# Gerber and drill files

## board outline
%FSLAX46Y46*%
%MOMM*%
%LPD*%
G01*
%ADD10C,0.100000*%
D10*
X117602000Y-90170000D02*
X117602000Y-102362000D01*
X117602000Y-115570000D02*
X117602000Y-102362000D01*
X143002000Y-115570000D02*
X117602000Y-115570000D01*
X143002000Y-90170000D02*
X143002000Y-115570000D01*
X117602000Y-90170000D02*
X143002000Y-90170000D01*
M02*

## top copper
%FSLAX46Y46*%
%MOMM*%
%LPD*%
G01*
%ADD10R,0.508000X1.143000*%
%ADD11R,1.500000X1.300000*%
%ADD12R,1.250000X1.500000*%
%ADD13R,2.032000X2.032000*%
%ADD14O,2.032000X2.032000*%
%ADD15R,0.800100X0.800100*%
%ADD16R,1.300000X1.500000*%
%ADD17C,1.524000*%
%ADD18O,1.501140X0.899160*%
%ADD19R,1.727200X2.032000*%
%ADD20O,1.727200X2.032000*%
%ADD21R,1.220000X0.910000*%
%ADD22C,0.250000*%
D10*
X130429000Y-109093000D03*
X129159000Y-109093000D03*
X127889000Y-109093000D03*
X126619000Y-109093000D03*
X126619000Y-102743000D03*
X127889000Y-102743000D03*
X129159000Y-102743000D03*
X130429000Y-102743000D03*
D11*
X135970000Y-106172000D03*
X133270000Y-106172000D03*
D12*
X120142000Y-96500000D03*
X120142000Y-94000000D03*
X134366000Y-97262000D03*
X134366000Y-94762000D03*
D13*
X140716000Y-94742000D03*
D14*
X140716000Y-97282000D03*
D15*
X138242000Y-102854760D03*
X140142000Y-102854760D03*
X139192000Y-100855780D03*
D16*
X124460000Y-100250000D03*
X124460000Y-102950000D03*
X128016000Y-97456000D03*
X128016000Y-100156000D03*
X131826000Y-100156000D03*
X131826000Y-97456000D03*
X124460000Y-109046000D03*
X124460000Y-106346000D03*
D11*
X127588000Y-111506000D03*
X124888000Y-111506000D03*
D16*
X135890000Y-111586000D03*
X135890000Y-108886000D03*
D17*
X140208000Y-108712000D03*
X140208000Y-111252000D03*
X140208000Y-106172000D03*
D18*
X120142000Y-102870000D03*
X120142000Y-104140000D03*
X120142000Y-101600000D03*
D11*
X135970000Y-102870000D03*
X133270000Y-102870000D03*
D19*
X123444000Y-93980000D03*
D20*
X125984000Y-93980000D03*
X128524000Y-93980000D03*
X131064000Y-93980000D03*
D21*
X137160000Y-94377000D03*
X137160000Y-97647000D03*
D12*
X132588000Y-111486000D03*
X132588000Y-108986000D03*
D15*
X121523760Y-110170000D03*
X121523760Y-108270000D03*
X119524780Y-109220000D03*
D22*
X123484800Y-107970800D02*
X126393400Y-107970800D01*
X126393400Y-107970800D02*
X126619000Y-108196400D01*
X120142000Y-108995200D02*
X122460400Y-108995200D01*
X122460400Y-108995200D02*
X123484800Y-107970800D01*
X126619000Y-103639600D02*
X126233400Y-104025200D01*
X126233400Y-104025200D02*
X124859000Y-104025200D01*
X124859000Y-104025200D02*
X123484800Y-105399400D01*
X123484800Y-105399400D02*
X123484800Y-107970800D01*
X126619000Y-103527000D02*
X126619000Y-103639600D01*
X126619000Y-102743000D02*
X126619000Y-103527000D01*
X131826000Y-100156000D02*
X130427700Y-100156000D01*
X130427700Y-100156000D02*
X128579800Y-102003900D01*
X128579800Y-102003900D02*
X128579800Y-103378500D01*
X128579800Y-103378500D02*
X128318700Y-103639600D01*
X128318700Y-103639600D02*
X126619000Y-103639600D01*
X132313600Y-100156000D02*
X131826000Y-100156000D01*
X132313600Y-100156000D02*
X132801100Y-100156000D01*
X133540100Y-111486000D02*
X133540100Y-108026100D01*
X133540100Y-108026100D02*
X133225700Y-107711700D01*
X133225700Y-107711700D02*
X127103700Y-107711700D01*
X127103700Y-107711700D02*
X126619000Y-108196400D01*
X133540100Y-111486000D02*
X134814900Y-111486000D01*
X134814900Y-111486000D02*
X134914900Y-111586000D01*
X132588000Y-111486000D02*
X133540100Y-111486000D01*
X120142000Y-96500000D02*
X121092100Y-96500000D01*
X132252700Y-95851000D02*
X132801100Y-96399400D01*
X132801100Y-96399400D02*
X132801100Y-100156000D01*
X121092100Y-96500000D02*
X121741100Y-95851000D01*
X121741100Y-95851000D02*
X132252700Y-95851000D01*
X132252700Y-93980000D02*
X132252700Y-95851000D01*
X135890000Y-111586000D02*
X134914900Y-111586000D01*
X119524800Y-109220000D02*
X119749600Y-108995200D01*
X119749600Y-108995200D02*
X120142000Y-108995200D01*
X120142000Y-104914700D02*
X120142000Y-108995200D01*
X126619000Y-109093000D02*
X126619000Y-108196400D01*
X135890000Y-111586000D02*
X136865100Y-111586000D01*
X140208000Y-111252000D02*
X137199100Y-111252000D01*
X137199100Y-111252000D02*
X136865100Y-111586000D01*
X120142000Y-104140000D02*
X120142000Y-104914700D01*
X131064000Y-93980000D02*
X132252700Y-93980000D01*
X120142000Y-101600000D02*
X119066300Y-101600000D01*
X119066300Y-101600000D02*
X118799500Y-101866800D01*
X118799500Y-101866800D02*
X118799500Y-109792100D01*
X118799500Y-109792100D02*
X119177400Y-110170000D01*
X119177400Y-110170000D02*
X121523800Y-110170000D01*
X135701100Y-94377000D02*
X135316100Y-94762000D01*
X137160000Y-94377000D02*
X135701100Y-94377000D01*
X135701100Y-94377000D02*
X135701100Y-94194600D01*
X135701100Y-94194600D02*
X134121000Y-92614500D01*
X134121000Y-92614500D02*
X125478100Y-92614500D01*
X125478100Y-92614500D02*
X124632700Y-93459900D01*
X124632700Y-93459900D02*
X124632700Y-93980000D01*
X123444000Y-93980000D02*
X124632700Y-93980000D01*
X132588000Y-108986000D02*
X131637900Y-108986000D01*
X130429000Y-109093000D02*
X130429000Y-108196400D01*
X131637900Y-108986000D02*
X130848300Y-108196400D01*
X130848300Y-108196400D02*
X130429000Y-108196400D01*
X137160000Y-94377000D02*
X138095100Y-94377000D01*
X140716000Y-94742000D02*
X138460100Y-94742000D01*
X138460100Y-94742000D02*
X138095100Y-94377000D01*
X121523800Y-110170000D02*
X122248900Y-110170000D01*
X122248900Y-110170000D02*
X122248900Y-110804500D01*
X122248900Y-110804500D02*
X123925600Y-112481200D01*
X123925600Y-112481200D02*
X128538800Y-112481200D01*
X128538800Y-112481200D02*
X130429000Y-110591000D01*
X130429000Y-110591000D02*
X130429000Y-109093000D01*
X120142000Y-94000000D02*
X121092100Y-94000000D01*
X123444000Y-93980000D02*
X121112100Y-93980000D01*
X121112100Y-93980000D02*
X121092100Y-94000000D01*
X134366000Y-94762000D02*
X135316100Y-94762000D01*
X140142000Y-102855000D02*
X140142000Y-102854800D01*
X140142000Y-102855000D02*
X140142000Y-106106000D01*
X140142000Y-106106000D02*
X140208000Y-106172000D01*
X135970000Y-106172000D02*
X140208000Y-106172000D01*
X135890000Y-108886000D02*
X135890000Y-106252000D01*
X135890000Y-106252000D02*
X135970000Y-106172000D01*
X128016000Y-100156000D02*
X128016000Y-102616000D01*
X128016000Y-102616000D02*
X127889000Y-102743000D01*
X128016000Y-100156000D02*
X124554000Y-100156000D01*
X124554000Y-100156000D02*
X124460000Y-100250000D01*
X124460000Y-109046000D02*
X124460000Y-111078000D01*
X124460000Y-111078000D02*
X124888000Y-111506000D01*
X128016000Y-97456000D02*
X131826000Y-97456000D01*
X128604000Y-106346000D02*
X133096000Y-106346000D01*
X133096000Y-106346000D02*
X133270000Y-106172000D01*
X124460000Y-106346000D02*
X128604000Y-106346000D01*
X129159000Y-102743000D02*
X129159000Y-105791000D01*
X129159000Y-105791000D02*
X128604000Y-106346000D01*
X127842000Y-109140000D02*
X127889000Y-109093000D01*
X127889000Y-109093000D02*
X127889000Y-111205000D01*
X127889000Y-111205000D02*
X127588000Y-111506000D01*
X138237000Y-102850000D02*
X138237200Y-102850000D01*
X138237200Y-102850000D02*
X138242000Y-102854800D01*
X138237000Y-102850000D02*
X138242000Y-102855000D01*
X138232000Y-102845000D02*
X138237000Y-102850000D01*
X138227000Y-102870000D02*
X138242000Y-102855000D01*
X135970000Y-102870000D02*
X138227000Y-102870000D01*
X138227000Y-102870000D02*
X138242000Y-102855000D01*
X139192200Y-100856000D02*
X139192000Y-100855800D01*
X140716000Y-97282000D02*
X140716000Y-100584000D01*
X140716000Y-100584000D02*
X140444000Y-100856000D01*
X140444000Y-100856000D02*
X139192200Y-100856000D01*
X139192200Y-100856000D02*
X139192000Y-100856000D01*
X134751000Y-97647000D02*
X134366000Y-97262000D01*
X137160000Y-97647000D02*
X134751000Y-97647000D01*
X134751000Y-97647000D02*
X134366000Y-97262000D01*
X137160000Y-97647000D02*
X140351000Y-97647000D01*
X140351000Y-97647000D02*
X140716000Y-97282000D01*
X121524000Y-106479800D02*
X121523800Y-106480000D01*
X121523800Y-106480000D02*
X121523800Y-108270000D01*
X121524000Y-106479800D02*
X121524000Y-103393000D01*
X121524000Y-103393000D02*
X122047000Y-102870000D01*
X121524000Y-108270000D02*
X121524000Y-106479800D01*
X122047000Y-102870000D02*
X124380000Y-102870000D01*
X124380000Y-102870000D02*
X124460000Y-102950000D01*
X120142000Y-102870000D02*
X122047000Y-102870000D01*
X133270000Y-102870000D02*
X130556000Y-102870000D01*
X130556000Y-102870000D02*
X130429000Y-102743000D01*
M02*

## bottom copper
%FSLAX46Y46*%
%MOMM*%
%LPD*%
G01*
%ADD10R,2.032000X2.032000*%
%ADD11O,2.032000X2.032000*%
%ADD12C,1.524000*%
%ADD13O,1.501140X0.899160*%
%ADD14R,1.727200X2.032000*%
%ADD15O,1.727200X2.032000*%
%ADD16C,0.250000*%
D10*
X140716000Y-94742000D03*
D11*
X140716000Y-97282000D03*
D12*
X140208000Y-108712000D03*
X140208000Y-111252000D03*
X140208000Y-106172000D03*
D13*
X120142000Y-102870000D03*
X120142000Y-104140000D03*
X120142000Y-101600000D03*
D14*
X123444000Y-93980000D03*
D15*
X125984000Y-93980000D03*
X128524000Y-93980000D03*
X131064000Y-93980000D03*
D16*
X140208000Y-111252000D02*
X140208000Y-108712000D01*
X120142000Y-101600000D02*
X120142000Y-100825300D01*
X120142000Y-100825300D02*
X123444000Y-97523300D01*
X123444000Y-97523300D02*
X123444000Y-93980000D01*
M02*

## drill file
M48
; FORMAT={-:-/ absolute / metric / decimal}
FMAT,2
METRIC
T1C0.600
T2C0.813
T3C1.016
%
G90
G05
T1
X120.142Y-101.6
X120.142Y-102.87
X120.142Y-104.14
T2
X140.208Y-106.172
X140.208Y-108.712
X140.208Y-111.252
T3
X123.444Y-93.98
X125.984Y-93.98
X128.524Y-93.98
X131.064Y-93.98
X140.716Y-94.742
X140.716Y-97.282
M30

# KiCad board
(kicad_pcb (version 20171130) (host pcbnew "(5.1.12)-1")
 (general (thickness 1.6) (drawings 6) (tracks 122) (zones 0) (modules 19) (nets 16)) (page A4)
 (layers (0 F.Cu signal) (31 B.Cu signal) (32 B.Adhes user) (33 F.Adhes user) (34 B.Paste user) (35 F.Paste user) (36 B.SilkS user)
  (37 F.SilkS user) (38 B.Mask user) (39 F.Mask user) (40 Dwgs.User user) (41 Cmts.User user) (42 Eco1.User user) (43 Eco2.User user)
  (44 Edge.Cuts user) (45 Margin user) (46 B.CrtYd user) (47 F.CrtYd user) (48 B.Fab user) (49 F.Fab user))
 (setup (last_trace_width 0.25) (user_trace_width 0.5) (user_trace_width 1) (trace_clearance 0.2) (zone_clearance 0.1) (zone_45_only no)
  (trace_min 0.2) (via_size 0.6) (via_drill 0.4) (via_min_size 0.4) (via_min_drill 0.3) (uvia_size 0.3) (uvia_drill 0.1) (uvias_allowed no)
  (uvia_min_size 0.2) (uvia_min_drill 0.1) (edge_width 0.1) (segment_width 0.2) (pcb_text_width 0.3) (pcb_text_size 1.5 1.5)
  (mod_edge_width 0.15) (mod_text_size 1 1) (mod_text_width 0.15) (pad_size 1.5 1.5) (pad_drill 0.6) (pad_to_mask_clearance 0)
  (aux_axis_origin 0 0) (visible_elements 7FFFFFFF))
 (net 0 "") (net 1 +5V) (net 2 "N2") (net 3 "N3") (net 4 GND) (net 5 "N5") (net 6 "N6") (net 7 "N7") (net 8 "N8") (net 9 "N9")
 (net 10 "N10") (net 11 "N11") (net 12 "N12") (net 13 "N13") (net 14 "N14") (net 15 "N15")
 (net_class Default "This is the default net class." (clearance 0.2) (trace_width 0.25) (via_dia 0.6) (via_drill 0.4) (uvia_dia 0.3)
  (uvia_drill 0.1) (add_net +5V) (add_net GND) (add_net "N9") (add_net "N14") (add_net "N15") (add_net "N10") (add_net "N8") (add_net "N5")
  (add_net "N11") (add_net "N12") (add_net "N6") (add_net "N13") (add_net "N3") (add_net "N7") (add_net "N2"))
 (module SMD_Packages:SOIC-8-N (layer F.Cu) (at 128.524 105.918 180)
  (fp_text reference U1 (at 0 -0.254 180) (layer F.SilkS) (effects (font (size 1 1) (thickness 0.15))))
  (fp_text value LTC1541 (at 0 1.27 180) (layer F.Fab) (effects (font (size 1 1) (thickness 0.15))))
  (pad 8 smd rect (at -1.905 -3.175 180) (size 0.508 1.143) (layers F.Cu F.Paste F.Mask) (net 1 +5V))
  (pad 7 smd rect (at -0.635 -3.175 180) (size 0.508 1.143) (layers F.Cu F.Paste F.Mask) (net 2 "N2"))
  (pad 6 smd rect (at 0.635 -3.175 180) (size 0.508 1.143) (layers F.Cu F.Paste F.Mask) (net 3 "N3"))
  (pad 5 smd rect (at 1.905 -3.175 180) (size 0.508 1.143) (layers F.Cu F.Paste F.Mask) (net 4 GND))
  (pad 4 smd rect (at 1.905 3.175 180) (size 0.508 1.143) (layers F.Cu F.Paste F.Mask) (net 4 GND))
  (pad 3 smd rect (at 0.635 3.175 180) (size 0.508 1.143) (layers F.Cu F.Paste F.Mask) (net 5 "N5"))
  (pad 2 smd rect (at -0.635 3.175 180) (size 0.508 1.143) (layers F.Cu F.Paste F.Mask) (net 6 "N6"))
  (pad 1 smd rect (at -1.905 3.175 180) (size 0.508 1.143) (layers F.Cu F.Paste F.Mask) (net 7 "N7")))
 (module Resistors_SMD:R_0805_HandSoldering (layer F.Cu) (at 134.62 106.172 180)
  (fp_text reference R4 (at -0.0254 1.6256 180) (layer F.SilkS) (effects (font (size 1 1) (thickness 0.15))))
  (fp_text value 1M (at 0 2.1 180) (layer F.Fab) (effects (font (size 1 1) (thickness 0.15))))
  (pad 1 smd rect (at -1.35 0 180) (size 1.5 1.3) (layers F.Cu F.Paste F.Mask) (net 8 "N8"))
  (pad 2 smd rect (at 1.35 0 180) (size 1.5 1.3) (layers F.Cu F.Paste F.Mask) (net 6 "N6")))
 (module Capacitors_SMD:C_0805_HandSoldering (layer F.Cu) (at 120.142 95.25 90)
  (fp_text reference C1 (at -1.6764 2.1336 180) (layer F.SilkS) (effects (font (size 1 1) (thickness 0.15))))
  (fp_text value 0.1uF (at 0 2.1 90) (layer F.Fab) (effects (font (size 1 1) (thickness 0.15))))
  (pad 1 smd rect (at -1.25 0 90) (size 1.5 1.25) (layers F.Cu F.Paste F.Mask) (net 4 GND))
  (pad 2 smd rect (at 1.25 0 90) (size 1.5 1.25) (layers F.Cu F.Paste F.Mask) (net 1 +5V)))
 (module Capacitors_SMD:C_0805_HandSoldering (layer F.Cu) (at 134.366 96.012 90)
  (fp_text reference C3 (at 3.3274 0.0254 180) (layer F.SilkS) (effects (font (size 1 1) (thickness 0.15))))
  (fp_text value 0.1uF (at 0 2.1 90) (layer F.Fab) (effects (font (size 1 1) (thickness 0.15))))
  (pad 1 smd rect (at -1.25 0 90) (size 1.5 1.25) (layers F.Cu F.Paste F.Mask) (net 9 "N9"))
  (pad 2 smd rect (at 1.25 0 90) (size 1.5 1.25) (layers F.Cu F.Paste F.Mask) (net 1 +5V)))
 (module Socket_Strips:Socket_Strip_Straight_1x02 (layer F.Cu) (at 140.716 94.742 270)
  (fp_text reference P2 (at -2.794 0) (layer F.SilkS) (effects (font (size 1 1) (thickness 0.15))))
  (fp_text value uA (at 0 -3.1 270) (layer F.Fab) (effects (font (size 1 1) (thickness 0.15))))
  (pad 1 thru_hole rect (at 0 0 270) (size 2.032 2.032) (drill 1.016) (layers *.Cu *.Mask F.SilkS) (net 1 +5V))
  (pad 2 thru_hole oval (at 2.54 0 270) (size 2.032 2.032) (drill 1.016) (layers *.Cu *.Mask F.SilkS) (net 9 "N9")))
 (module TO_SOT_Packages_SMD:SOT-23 (layer F.Cu) (at 139.192 101.854)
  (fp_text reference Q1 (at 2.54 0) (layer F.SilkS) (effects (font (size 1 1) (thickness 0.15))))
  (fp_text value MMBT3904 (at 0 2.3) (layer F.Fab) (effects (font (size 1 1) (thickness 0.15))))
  (pad 1 smd rect (at -0.95 1.00076) (size 0.8001 0.8001) (layers F.Cu F.Paste F.Mask) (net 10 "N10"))
  (pad 2 smd rect (at 0.95 1.00076) (size 0.8001 0.8001) (layers F.Cu F.Paste F.Mask) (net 8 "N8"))
  (pad 3 smd rect (at 0 -0.99822) (size 0.8001 0.8001) (layers F.Cu F.Paste F.Mask) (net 9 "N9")))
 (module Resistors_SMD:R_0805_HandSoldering (layer F.Cu) (at 124.46 101.6 270)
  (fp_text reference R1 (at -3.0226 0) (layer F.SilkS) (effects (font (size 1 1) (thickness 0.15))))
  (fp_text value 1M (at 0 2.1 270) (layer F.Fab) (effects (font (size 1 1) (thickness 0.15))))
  (pad 1 smd rect (at -1.35 0 270) (size 1.5 1.3) (layers F.Cu F.Paste F.Mask) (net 5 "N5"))
  (pad 2 smd rect (at 1.35 0 270) (size 1.5 1.3) (layers F.Cu F.Paste F.Mask) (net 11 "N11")))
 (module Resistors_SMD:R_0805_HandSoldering (layer F.Cu) (at 128.016 98.806 270)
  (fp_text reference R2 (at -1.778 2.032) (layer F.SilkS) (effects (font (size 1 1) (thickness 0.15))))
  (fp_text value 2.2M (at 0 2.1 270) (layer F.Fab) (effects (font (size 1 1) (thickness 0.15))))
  (pad 1 smd rect (at -1.35 0 270) (size 1.5 1.3) (layers F.Cu F.Paste F.Mask) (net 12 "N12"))
  (pad 2 smd rect (at 1.35 0 270) (size 1.5 1.3) (layers F.Cu F.Paste F.Mask) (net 5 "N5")))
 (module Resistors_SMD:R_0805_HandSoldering (layer F.Cu) (at 131.826 98.806 90)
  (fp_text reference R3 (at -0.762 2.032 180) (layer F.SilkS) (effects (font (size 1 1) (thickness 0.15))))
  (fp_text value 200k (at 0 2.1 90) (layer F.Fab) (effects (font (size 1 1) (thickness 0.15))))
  (pad 1 smd rect (at -1.35 0 90) (size 1.5 1.3) (layers F.Cu F.Paste F.Mask) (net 4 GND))
  (pad 2 smd rect (at 1.35 0 90) (size 1.5 1.3) (layers F.Cu F.Paste F.Mask) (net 12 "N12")))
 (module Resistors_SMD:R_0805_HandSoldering (layer F.Cu) (at 124.46 107.696 90)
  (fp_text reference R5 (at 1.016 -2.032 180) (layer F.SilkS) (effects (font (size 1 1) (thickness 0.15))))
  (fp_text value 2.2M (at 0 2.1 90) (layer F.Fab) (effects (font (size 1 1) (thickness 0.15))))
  (pad 1 smd rect (at -1.35 0 90) (size 1.5 1.3) (layers F.Cu F.Paste F.Mask) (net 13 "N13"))
  (pad 2 smd rect (at 1.35 0 90) (size 1.5 1.3) (layers F.Cu F.Paste F.Mask) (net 6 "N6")))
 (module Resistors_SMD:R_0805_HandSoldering (layer F.Cu) (at 126.238 111.506 180)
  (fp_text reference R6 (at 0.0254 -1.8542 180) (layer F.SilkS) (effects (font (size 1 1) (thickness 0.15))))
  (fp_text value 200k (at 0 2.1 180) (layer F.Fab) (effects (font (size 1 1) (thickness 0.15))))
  (pad 1 smd rect (at -1.35 0 180) (size 1.5 1.3) (layers F.Cu F.Paste F.Mask) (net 3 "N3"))
  (pad 2 smd rect (at 1.35 0 180) (size 1.5 1.3) (layers F.Cu F.Paste F.Mask) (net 13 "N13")))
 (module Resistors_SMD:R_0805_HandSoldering (layer F.Cu) (at 135.89 110.236 90)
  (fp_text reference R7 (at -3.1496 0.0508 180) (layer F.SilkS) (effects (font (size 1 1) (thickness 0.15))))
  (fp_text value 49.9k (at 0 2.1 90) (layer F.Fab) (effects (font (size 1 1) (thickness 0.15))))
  (pad 1 smd rect (at -1.35 0 90) (size 1.5 1.3) (layers F.Cu F.Paste F.Mask) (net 4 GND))
  (pad 2 smd rect (at 1.35 0 90) (size 1.5 1.3) (layers F.Cu F.Paste F.Mask) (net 8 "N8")))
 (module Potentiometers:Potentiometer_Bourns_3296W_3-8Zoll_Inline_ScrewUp (layer F.Cu) (at 140.208 106.172 180)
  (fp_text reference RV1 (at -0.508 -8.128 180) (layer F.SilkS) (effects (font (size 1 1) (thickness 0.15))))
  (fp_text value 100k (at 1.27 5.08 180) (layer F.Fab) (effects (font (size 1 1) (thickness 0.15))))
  (pad 2 thru_hole circle (at 0 -2.54 180) (size 1.524 1.524) (drill 0.8128) (layers *.Cu *.Mask F.SilkS) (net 4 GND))
  (pad 3 thru_hole circle (at 0 -5.08 180) (size 1.524 1.524) (drill 0.8128) (layers *.Cu *.Mask F.SilkS) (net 4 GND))
  (pad 1 thru_hole circle (at 0 0 180) (size 1.524 1.524) (drill 0.8128) (layers *.Cu *.Mask F.SilkS) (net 8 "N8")))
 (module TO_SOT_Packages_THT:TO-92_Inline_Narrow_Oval (layer F.Cu) (at 120.142 101.6 270)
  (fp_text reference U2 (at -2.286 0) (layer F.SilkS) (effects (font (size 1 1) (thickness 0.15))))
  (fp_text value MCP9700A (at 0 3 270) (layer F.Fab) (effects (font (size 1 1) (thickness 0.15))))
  (pad 2 thru_hole oval (at 1.27 0 90) (size 0.89916 1.50114) (drill 0.6) (layers *.Cu *.Mask F.SilkS) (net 11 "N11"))
  (pad 3 thru_hole oval (at 2.54 0 90) (size 0.89916 1.50114) (drill 0.6) (layers *.Cu *.Mask F.SilkS) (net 4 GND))
  (pad 1 thru_hole oval (at 0 0 90) (size 0.89916 1.50114) (drill 0.6) (layers *.Cu *.Mask F.SilkS) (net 1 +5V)))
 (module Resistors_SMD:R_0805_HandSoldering (layer F.Cu) (at 134.62 102.87 180)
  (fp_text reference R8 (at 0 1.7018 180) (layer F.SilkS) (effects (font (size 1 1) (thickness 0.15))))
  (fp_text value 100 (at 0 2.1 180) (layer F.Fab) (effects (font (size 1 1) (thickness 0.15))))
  (pad 1 smd rect (at -1.35 0 180) (size 1.5 1.3) (layers F.Cu F.Paste F.Mask) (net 10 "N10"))
  (pad 2 smd rect (at 1.35 0 180) (size 1.5 1.3) (layers F.Cu F.Paste F.Mask) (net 7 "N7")))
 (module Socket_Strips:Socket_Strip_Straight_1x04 (layer F.Cu) (at 123.444 93.98)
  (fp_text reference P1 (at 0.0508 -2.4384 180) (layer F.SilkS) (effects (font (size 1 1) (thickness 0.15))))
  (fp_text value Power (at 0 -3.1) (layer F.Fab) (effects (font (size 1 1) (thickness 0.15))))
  (pad 1 thru_hole rect (at 0 0) (size 1.7272 2.032) (drill 1.016) (layers *.Cu *.Mask F.SilkS) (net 1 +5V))
  (pad 2 thru_hole oval (at 2.54 0) (size 1.7272 2.032) (drill 1.016) (layers *.Cu *.Mask F.SilkS) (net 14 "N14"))
  (pad 3 thru_hole oval (at 5.08 0) (size 1.7272 2.032) (drill 1.016) (layers *.Cu *.Mask F.SilkS) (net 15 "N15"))
  (pad 4 thru_hole oval (at 7.62 0) (size 1.7272 2.032) (drill 1.016) (layers *.Cu *.Mask F.SilkS) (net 4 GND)))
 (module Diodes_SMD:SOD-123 (layer F.Cu) (at 137.16 96.012 270)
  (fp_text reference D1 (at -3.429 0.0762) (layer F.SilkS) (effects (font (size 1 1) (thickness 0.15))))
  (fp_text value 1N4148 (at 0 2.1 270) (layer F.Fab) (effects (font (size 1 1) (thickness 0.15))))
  (pad 1 smd rect (at -1.635 0 270) (size 0.91 1.22) (layers F.Cu F.Paste F.Mask) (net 1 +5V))
  (pad 2 smd rect (at 1.635 0 270) (size 0.91 1.22) (layers F.Cu F.Paste F.Mask) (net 9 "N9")))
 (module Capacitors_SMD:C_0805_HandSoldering (layer F.Cu) (at 132.588 110.236 90)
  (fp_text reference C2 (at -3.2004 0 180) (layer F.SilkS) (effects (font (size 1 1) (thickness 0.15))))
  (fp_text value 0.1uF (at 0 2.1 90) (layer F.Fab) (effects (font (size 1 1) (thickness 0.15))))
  (pad 1 smd rect (at -1.25 0 90) (size 1.5 1.25) (layers F.Cu F.Paste F.Mask) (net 4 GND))
  (pad 2 smd rect (at 1.25 0 90) (size 1.5 1.25) (layers F.Cu F.Paste F.Mask) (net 1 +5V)))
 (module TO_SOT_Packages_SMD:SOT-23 (layer F.Cu) (at 120.523 109.22 90)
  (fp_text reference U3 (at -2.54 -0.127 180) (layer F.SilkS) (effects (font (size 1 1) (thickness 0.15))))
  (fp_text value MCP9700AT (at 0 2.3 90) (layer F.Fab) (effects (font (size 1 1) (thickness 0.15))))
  (pad 1 smd rect (at -0.95 1.00076 90) (size 0.8001 0.8001) (layers F.Cu F.Paste F.Mask) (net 1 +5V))
  (pad 2 smd rect (at 0.95 1.00076 90) (size 0.8001 0.8001) (layers F.Cu F.Paste F.Mask) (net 11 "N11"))
  (pad 3 smd rect (at 0 -0.99822 90) (size 0.8001 0.8001) (layers F.Cu F.Paste F.Mask) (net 4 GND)))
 (gr_line (start 117.602 90.17) (end 117.602 102.362) (angle 90) (layer Edge.Cuts) (width 0.1))
 (gr_line (start 117.602 115.57) (end 117.602 102.362) (angle 90) (layer Edge.Cuts) (width 0.1))
 (gr_line (start 143.002 115.57) (end 117.602 115.57) (angle 90) (layer Edge.Cuts) (width 0.1))
 (gr_line (start 143.002 90.17) (end 143.002 115.57) (angle 90) (layer Edge.Cuts) (width 0.1))
 (gr_line (start 117.602 90.17) (end 143.002 90.17) (angle 90) (layer Edge.Cuts) (width 0.1))
 (segment (start 123.4848 107.9708) (end 126.3934 107.9708) (width 0.25) (layer F.Cu) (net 4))
 (segment (start 126.3934 107.9708) (end 126.619 108.1964) (width 0.25) (layer F.Cu) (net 4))
 (segment (start 120.142 108.9952) (end 122.4604 108.9952) (width 0.25) (layer F.Cu) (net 4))
 (segment (start 122.4604 108.9952) (end 123.4848 107.9708) (width 0.25) (layer F.Cu) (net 4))
 (segment (start 126.619 103.6396) (end 126.2334 104.0252) (width 0.25) (layer F.Cu) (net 4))
 (segment (start 126.2334 104.0252) (end 124.859 104.0252) (width 0.25) (layer F.Cu) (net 4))
 (segment (start 124.859 104.0252) (end 123.4848 105.3994) (width 0.25) (layer F.Cu) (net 4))
 (segment (start 123.4848 105.3994) (end 123.4848 107.9708) (width 0.25) (layer F.Cu) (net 4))
 (segment (start 126.619 103.527) (end 126.619 103.6396) (width 0.25) (layer F.Cu) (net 4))
 (segment (start 126.619 102.743) (end 126.619 103.527) (width 0.25) (layer F.Cu) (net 4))
 (segment (start 131.826 100.156) (end 130.4277 100.156) (width 0.25) (layer F.Cu) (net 4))
 (segment (start 130.4277 100.156) (end 128.5798 102.0039) (width 0.25) (layer F.Cu) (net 4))
 (segment (start 128.5798 102.0039) (end 128.5798 103.3785) (width 0.25) (layer F.Cu) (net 4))
 (segment (start 128.5798 103.3785) (end 128.3187 103.6396) (width 0.25) (layer F.Cu) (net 4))
 (segment (start 128.3187 103.6396) (end 126.619 103.6396) (width 0.25) (layer F.Cu) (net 4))
 (segment (start 132.3136 100.156) (end 131.826 100.156) (width 0.25) (layer F.Cu) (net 4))
 (segment (start 132.3136 100.156) (end 132.8011 100.156) (width 0.25) (layer F.Cu) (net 4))
 (segment (start 133.5401 111.486) (end 133.5401 108.0261) (width 0.25) (layer F.Cu) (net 4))
 (segment (start 133.5401 108.0261) (end 133.2257 107.7117) (width 0.25) (layer F.Cu) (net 4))
 (segment (start 133.2257 107.7117) (end 127.1037 107.7117) (width 0.25) (layer F.Cu) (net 4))
 (segment (start 127.1037 107.7117) (end 126.619 108.1964) (width 0.25) (layer F.Cu) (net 4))
 (segment (start 133.5401 111.486) (end 134.8149 111.486) (width 0.25) (layer F.Cu) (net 4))
 (segment (start 134.8149 111.486) (end 134.9149 111.586) (width 0.25) (layer F.Cu) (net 4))
 (segment (start 132.588 111.486) (end 133.5401 111.486) (width 0.25) (layer F.Cu) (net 4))
 (segment (start 120.142 96.5) (end 121.0921 96.5) (width 0.25) (layer F.Cu) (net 4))
 (segment (start 132.2527 95.851) (end 132.8011 96.3994) (width 0.25) (layer F.Cu) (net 4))
 (segment (start 132.8011 96.3994) (end 132.8011 100.156) (width 0.25) (layer F.Cu) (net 4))
 (segment (start 121.0921 96.5) (end 121.7411 95.851) (width 0.25) (layer F.Cu) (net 4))
 (segment (start 121.7411 95.851) (end 132.2527 95.851) (width 0.25) (layer F.Cu) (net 4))
 (segment (start 132.2527 93.98) (end 132.2527 95.851) (width 0.25) (layer F.Cu) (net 4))
 (segment (start 135.89 111.586) (end 134.9149 111.586) (width 0.25) (layer F.Cu) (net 4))
 (segment (start 119.5248 109.22) (end 119.7496 108.9952) (width 0.25) (layer F.Cu) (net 4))
 (segment (start 119.7496 108.9952) (end 120.142 108.9952) (width 0.25) (layer F.Cu) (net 4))
 (segment (start 120.142 104.9147) (end 120.142 108.9952) (width 0.25) (layer F.Cu) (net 4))
 (segment (start 126.619 109.093) (end 126.619 108.1964) (width 0.25) (layer F.Cu) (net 4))
 (segment (start 135.89 111.586) (end 136.8651 111.586) (width 0.25) (layer F.Cu) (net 4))
 (segment (start 140.208 111.252) (end 137.1991 111.252) (width 0.25) (layer F.Cu) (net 4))
 (segment (start 137.1991 111.252) (end 136.8651 111.586) (width 0.25) (layer F.Cu) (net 4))
 (segment (start 140.208 111.252) (end 140.208 108.712) (width 0.25) (layer B.Cu) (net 4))
 (segment (start 120.142 104.14) (end 120.142 104.9147) (width 0.25) (layer F.Cu) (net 4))
 (segment (start 131.064 93.98) (end 132.2527 93.98) (width 0.25) (layer F.Cu) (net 4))
 (segment (start 120.142 101.6) (end 119.0663 101.6) (width 0.25) (layer F.Cu) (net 1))
 (segment (start 119.0663 101.6) (end 118.7995 101.8668) (width 0.25) (layer F.Cu) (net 1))
 (segment (start 118.7995 101.8668) (end 118.7995 109.7921) (width 0.25) (layer F.Cu) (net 1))
 (segment (start 118.7995 109.7921) (end 119.1774 110.17) (width 0.25) (layer F.Cu) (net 1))
 (segment (start 119.1774 110.17) (end 121.5238 110.17) (width 0.25) (layer F.Cu) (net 1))
 (segment (start 135.7011 94.377) (end 135.3161 94.762) (width 0.25) (layer F.Cu) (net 1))
 (segment (start 137.16 94.377) (end 135.7011 94.377) (width 0.25) (layer F.Cu) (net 1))
 (segment (start 135.7011 94.377) (end 135.7011 94.1946) (width 0.25) (layer F.Cu) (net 1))
 (segment (start 135.7011 94.1946) (end 134.121 92.6145) (width 0.25) (layer F.Cu) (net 1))
 (segment (start 134.121 92.6145) (end 125.4781 92.6145) (width 0.25) (layer F.Cu) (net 1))
 (segment (start 125.4781 92.6145) (end 124.6327 93.4599) (width 0.25) (layer F.Cu) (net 1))
 (segment (start 124.6327 93.4599) (end 124.6327 93.98) (width 0.25) (layer F.Cu) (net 1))
 (segment (start 123.444 93.98) (end 124.6327 93.98) (width 0.25) (layer F.Cu) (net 1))
 (segment (start 132.588 108.986) (end 131.6379 108.986) (width 0.25) (layer F.Cu) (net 1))
 (segment (start 130.429 109.093) (end 130.429 108.1964) (width 0.25) (layer F.Cu) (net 1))
 (segment (start 131.6379 108.986) (end 130.8483 108.1964) (width 0.25) (layer F.Cu) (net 1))
 (segment (start 130.8483 108.1964) (end 130.429 108.1964) (width 0.25) (layer F.Cu) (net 1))
 (segment (start 137.16 94.377) (end 138.0951 94.377) (width 0.25) (layer F.Cu) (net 1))
 (segment (start 140.716 94.742) (end 138.4601 94.742) (width 0.25) (layer F.Cu) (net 1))
 (segment (start 138.4601 94.742) (end 138.0951 94.377) (width 0.25) (layer F.Cu) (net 1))
 (segment (start 121.5238 110.17) (end 122.2489 110.17) (width 0.25) (layer F.Cu) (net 1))
 (segment (start 122.2489 110.17) (end 122.2489 110.8045) (width 0.25) (layer F.Cu) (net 1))
 (segment (start 122.2489 110.8045) (end 123.9256 112.4812) (width 0.25) (layer F.Cu) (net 1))
 (segment (start 123.9256 112.4812) (end 128.5388 112.4812) (width 0.25) (layer F.Cu) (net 1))
 (segment (start 128.5388 112.4812) (end 130.429 110.591) (width 0.25) (layer F.Cu) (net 1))
 (segment (start 130.429 110.591) (end 130.429 109.093) (width 0.25) (layer F.Cu) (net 1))
 (segment (start 120.142 101.6) (end 120.142 100.8253) (width 0.25) (layer B.Cu) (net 1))
 (segment (start 120.142 100.8253) (end 123.444 97.5233) (width 0.25) (layer B.Cu) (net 1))
 (segment (start 123.444 97.5233) (end 123.444 93.98) (width 0.25) (layer B.Cu) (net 1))
 (segment (start 120.142 94) (end 121.0921 94) (width 0.25) (layer F.Cu) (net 1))
 (segment (start 123.444 93.98) (end 121.1121 93.98) (width 0.25) (layer F.Cu) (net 1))
 (segment (start 121.1121 93.98) (end 121.0921 94) (width 0.25) (layer F.Cu) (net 1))
 (segment (start 134.366 94.762) (end 135.3161 94.762) (width 0.25) (layer F.Cu) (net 1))
 (segment (start 140.142 102.855) (end 140.142 102.8548) (width 0.25) (layer F.Cu) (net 8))
 (segment (start 140.142 102.855) (end 140.142 106.106) (width 0.25) (layer F.Cu) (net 8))
 (segment (start 140.142 106.106) (end 140.208 106.172) (width 0.25) (layer F.Cu) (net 8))
 (segment (start 135.97 106.172) (end 140.208 106.172) (width 0.25) (layer F.Cu) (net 8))
 (segment (start 135.89 108.886) (end 135.89 106.252) (width 0.25) (layer F.Cu) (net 8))
 (segment (start 135.89 106.252) (end 135.97 106.172) (width 0.25) (layer F.Cu) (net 8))
 (segment (start 128.016 100.156) (end 128.016 102.616) (width 0.25) (layer F.Cu) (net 5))
 (segment (start 128.016 102.616) (end 127.889 102.743) (width 0.25) (layer F.Cu) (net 5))
 (segment (start 128.016 100.156) (end 124.554 100.156) (width 0.25) (layer F.Cu) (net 5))
 (segment (start 124.554 100.156) (end 124.46 100.25) (width 0.25) (layer F.Cu) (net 5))
 (segment (start 124.46 109.046) (end 124.46 111.078) (width 0.25) (layer F.Cu) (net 13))
 (segment (start 124.46 111.078) (end 124.888 111.506) (width 0.25) (layer F.Cu) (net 13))
 (segment (start 128.016 97.456) (end 131.826 97.456) (width 0.25) (layer F.Cu) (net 12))
 (segment (start 128.604 106.346) (end 133.096 106.346) (width 0.25) (layer F.Cu) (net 6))
 (segment (start 133.096 106.346) (end 133.27 106.172) (width 0.25) (layer F.Cu) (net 6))
 (segment (start 124.46 106.346) (end 128.604 106.346) (width 0.25) (layer F.Cu) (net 6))
 (segment (start 129.159 102.743) (end 129.159 105.791) (width 0.25) (layer F.Cu) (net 6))
 (segment (start 129.159 105.791) (end 128.604 106.346) (width 0.25) (layer F.Cu) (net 6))
 (segment (start 127.842 109.14) (end 127.889 109.093) (width 0.25) (layer F.Cu) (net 3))
 (segment (start 127.889 109.093) (end 127.889 111.205) (width 0.25) (layer F.Cu) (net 3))
 (segment (start 127.889 111.205) (end 127.588 111.506) (width 0.25) (layer F.Cu) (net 3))
 (segment (start 138.237 102.85) (end 138.2372 102.85) (width 0.25) (layer F.Cu) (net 10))
 (segment (start 138.2372 102.85) (end 138.242 102.8548) (width 0.25) (layer F.Cu) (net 10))
 (segment (start 138.237 102.85) (end 138.242 102.855) (width 0.25) (layer F.Cu) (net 10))
 (segment (start 138.232 102.845) (end 138.237 102.85) (width 0.25) (layer F.Cu) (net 10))
 (segment (start 138.227 102.87) (end 138.242 102.855) (width 0.25) (layer F.Cu) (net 10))
 (segment (start 135.97 102.87) (end 138.227 102.87) (width 0.25) (layer F.Cu) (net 10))
 (segment (start 138.227 102.87) (end 138.242 102.855) (width 0.25) (layer F.Cu) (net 10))
 (segment (start 139.1922 100.856) (end 139.192 100.8558) (width 0.25) (layer F.Cu) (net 9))
 (segment (start 140.716 97.282) (end 140.716 100.584) (width 0.25) (layer F.Cu) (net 9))
 (segment (start 140.716 100.584) (end 140.444 100.856) (width 0.25) (layer F.Cu) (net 9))
 (segment (start 140.444 100.856) (end 139.1922 100.856) (width 0.25) (layer F.Cu) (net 9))
 (segment (start 139.1922 100.856) (end 139.192 100.856) (width 0.25) (layer F.Cu) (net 9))
 (segment (start 134.751 97.647) (end 134.366 97.262) (width 0.25) (layer F.Cu) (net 9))
 (segment (start 137.16 97.647) (end 134.751 97.647) (width 0.25) (layer F.Cu) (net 9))
 (segment (start 134.751 97.647) (end 134.366 97.262) (width 0.25) (layer F.Cu) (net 9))
 (segment (start 137.16 97.647) (end 140.351 97.647) (width 0.25) (layer F.Cu) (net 9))
 (segment (start 140.351 97.647) (end 140.716 97.282) (width 0.25) (layer F.Cu) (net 9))
 (segment (start 121.524 106.4798) (end 121.5238 106.48) (width 0.25) (layer F.Cu) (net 11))
 (segment (start 121.5238 106.48) (end 121.5238 108.27) (width 0.25) (layer F.Cu) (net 11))
 (segment (start 121.524 106.4798) (end 121.524 103.393) (width 0.25) (layer F.Cu) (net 11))
 (segment (start 121.524 103.393) (end 122.047 102.87) (width 0.25) (layer F.Cu) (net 11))
 (segment (start 121.524 108.27) (end 121.524 106.4798) (width 0.25) (layer F.Cu) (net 11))
 (segment (start 122.047 102.87) (end 124.38 102.87) (width 0.25) (layer F.Cu) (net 11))
 (segment (start 124.38 102.87) (end 124.46 102.95) (width 0.25) (layer F.Cu) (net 11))
 (segment (start 120.142 102.87) (end 122.047 102.87) (width 0.25) (layer F.Cu) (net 11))
 (segment (start 133.27 102.87) (end 130.556 102.87) (width 0.25) (layer F.Cu) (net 7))
 (segment (start 130.556 102.87) (end 130.429 102.743) (width 0.25) (layer F.Cu) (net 7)))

